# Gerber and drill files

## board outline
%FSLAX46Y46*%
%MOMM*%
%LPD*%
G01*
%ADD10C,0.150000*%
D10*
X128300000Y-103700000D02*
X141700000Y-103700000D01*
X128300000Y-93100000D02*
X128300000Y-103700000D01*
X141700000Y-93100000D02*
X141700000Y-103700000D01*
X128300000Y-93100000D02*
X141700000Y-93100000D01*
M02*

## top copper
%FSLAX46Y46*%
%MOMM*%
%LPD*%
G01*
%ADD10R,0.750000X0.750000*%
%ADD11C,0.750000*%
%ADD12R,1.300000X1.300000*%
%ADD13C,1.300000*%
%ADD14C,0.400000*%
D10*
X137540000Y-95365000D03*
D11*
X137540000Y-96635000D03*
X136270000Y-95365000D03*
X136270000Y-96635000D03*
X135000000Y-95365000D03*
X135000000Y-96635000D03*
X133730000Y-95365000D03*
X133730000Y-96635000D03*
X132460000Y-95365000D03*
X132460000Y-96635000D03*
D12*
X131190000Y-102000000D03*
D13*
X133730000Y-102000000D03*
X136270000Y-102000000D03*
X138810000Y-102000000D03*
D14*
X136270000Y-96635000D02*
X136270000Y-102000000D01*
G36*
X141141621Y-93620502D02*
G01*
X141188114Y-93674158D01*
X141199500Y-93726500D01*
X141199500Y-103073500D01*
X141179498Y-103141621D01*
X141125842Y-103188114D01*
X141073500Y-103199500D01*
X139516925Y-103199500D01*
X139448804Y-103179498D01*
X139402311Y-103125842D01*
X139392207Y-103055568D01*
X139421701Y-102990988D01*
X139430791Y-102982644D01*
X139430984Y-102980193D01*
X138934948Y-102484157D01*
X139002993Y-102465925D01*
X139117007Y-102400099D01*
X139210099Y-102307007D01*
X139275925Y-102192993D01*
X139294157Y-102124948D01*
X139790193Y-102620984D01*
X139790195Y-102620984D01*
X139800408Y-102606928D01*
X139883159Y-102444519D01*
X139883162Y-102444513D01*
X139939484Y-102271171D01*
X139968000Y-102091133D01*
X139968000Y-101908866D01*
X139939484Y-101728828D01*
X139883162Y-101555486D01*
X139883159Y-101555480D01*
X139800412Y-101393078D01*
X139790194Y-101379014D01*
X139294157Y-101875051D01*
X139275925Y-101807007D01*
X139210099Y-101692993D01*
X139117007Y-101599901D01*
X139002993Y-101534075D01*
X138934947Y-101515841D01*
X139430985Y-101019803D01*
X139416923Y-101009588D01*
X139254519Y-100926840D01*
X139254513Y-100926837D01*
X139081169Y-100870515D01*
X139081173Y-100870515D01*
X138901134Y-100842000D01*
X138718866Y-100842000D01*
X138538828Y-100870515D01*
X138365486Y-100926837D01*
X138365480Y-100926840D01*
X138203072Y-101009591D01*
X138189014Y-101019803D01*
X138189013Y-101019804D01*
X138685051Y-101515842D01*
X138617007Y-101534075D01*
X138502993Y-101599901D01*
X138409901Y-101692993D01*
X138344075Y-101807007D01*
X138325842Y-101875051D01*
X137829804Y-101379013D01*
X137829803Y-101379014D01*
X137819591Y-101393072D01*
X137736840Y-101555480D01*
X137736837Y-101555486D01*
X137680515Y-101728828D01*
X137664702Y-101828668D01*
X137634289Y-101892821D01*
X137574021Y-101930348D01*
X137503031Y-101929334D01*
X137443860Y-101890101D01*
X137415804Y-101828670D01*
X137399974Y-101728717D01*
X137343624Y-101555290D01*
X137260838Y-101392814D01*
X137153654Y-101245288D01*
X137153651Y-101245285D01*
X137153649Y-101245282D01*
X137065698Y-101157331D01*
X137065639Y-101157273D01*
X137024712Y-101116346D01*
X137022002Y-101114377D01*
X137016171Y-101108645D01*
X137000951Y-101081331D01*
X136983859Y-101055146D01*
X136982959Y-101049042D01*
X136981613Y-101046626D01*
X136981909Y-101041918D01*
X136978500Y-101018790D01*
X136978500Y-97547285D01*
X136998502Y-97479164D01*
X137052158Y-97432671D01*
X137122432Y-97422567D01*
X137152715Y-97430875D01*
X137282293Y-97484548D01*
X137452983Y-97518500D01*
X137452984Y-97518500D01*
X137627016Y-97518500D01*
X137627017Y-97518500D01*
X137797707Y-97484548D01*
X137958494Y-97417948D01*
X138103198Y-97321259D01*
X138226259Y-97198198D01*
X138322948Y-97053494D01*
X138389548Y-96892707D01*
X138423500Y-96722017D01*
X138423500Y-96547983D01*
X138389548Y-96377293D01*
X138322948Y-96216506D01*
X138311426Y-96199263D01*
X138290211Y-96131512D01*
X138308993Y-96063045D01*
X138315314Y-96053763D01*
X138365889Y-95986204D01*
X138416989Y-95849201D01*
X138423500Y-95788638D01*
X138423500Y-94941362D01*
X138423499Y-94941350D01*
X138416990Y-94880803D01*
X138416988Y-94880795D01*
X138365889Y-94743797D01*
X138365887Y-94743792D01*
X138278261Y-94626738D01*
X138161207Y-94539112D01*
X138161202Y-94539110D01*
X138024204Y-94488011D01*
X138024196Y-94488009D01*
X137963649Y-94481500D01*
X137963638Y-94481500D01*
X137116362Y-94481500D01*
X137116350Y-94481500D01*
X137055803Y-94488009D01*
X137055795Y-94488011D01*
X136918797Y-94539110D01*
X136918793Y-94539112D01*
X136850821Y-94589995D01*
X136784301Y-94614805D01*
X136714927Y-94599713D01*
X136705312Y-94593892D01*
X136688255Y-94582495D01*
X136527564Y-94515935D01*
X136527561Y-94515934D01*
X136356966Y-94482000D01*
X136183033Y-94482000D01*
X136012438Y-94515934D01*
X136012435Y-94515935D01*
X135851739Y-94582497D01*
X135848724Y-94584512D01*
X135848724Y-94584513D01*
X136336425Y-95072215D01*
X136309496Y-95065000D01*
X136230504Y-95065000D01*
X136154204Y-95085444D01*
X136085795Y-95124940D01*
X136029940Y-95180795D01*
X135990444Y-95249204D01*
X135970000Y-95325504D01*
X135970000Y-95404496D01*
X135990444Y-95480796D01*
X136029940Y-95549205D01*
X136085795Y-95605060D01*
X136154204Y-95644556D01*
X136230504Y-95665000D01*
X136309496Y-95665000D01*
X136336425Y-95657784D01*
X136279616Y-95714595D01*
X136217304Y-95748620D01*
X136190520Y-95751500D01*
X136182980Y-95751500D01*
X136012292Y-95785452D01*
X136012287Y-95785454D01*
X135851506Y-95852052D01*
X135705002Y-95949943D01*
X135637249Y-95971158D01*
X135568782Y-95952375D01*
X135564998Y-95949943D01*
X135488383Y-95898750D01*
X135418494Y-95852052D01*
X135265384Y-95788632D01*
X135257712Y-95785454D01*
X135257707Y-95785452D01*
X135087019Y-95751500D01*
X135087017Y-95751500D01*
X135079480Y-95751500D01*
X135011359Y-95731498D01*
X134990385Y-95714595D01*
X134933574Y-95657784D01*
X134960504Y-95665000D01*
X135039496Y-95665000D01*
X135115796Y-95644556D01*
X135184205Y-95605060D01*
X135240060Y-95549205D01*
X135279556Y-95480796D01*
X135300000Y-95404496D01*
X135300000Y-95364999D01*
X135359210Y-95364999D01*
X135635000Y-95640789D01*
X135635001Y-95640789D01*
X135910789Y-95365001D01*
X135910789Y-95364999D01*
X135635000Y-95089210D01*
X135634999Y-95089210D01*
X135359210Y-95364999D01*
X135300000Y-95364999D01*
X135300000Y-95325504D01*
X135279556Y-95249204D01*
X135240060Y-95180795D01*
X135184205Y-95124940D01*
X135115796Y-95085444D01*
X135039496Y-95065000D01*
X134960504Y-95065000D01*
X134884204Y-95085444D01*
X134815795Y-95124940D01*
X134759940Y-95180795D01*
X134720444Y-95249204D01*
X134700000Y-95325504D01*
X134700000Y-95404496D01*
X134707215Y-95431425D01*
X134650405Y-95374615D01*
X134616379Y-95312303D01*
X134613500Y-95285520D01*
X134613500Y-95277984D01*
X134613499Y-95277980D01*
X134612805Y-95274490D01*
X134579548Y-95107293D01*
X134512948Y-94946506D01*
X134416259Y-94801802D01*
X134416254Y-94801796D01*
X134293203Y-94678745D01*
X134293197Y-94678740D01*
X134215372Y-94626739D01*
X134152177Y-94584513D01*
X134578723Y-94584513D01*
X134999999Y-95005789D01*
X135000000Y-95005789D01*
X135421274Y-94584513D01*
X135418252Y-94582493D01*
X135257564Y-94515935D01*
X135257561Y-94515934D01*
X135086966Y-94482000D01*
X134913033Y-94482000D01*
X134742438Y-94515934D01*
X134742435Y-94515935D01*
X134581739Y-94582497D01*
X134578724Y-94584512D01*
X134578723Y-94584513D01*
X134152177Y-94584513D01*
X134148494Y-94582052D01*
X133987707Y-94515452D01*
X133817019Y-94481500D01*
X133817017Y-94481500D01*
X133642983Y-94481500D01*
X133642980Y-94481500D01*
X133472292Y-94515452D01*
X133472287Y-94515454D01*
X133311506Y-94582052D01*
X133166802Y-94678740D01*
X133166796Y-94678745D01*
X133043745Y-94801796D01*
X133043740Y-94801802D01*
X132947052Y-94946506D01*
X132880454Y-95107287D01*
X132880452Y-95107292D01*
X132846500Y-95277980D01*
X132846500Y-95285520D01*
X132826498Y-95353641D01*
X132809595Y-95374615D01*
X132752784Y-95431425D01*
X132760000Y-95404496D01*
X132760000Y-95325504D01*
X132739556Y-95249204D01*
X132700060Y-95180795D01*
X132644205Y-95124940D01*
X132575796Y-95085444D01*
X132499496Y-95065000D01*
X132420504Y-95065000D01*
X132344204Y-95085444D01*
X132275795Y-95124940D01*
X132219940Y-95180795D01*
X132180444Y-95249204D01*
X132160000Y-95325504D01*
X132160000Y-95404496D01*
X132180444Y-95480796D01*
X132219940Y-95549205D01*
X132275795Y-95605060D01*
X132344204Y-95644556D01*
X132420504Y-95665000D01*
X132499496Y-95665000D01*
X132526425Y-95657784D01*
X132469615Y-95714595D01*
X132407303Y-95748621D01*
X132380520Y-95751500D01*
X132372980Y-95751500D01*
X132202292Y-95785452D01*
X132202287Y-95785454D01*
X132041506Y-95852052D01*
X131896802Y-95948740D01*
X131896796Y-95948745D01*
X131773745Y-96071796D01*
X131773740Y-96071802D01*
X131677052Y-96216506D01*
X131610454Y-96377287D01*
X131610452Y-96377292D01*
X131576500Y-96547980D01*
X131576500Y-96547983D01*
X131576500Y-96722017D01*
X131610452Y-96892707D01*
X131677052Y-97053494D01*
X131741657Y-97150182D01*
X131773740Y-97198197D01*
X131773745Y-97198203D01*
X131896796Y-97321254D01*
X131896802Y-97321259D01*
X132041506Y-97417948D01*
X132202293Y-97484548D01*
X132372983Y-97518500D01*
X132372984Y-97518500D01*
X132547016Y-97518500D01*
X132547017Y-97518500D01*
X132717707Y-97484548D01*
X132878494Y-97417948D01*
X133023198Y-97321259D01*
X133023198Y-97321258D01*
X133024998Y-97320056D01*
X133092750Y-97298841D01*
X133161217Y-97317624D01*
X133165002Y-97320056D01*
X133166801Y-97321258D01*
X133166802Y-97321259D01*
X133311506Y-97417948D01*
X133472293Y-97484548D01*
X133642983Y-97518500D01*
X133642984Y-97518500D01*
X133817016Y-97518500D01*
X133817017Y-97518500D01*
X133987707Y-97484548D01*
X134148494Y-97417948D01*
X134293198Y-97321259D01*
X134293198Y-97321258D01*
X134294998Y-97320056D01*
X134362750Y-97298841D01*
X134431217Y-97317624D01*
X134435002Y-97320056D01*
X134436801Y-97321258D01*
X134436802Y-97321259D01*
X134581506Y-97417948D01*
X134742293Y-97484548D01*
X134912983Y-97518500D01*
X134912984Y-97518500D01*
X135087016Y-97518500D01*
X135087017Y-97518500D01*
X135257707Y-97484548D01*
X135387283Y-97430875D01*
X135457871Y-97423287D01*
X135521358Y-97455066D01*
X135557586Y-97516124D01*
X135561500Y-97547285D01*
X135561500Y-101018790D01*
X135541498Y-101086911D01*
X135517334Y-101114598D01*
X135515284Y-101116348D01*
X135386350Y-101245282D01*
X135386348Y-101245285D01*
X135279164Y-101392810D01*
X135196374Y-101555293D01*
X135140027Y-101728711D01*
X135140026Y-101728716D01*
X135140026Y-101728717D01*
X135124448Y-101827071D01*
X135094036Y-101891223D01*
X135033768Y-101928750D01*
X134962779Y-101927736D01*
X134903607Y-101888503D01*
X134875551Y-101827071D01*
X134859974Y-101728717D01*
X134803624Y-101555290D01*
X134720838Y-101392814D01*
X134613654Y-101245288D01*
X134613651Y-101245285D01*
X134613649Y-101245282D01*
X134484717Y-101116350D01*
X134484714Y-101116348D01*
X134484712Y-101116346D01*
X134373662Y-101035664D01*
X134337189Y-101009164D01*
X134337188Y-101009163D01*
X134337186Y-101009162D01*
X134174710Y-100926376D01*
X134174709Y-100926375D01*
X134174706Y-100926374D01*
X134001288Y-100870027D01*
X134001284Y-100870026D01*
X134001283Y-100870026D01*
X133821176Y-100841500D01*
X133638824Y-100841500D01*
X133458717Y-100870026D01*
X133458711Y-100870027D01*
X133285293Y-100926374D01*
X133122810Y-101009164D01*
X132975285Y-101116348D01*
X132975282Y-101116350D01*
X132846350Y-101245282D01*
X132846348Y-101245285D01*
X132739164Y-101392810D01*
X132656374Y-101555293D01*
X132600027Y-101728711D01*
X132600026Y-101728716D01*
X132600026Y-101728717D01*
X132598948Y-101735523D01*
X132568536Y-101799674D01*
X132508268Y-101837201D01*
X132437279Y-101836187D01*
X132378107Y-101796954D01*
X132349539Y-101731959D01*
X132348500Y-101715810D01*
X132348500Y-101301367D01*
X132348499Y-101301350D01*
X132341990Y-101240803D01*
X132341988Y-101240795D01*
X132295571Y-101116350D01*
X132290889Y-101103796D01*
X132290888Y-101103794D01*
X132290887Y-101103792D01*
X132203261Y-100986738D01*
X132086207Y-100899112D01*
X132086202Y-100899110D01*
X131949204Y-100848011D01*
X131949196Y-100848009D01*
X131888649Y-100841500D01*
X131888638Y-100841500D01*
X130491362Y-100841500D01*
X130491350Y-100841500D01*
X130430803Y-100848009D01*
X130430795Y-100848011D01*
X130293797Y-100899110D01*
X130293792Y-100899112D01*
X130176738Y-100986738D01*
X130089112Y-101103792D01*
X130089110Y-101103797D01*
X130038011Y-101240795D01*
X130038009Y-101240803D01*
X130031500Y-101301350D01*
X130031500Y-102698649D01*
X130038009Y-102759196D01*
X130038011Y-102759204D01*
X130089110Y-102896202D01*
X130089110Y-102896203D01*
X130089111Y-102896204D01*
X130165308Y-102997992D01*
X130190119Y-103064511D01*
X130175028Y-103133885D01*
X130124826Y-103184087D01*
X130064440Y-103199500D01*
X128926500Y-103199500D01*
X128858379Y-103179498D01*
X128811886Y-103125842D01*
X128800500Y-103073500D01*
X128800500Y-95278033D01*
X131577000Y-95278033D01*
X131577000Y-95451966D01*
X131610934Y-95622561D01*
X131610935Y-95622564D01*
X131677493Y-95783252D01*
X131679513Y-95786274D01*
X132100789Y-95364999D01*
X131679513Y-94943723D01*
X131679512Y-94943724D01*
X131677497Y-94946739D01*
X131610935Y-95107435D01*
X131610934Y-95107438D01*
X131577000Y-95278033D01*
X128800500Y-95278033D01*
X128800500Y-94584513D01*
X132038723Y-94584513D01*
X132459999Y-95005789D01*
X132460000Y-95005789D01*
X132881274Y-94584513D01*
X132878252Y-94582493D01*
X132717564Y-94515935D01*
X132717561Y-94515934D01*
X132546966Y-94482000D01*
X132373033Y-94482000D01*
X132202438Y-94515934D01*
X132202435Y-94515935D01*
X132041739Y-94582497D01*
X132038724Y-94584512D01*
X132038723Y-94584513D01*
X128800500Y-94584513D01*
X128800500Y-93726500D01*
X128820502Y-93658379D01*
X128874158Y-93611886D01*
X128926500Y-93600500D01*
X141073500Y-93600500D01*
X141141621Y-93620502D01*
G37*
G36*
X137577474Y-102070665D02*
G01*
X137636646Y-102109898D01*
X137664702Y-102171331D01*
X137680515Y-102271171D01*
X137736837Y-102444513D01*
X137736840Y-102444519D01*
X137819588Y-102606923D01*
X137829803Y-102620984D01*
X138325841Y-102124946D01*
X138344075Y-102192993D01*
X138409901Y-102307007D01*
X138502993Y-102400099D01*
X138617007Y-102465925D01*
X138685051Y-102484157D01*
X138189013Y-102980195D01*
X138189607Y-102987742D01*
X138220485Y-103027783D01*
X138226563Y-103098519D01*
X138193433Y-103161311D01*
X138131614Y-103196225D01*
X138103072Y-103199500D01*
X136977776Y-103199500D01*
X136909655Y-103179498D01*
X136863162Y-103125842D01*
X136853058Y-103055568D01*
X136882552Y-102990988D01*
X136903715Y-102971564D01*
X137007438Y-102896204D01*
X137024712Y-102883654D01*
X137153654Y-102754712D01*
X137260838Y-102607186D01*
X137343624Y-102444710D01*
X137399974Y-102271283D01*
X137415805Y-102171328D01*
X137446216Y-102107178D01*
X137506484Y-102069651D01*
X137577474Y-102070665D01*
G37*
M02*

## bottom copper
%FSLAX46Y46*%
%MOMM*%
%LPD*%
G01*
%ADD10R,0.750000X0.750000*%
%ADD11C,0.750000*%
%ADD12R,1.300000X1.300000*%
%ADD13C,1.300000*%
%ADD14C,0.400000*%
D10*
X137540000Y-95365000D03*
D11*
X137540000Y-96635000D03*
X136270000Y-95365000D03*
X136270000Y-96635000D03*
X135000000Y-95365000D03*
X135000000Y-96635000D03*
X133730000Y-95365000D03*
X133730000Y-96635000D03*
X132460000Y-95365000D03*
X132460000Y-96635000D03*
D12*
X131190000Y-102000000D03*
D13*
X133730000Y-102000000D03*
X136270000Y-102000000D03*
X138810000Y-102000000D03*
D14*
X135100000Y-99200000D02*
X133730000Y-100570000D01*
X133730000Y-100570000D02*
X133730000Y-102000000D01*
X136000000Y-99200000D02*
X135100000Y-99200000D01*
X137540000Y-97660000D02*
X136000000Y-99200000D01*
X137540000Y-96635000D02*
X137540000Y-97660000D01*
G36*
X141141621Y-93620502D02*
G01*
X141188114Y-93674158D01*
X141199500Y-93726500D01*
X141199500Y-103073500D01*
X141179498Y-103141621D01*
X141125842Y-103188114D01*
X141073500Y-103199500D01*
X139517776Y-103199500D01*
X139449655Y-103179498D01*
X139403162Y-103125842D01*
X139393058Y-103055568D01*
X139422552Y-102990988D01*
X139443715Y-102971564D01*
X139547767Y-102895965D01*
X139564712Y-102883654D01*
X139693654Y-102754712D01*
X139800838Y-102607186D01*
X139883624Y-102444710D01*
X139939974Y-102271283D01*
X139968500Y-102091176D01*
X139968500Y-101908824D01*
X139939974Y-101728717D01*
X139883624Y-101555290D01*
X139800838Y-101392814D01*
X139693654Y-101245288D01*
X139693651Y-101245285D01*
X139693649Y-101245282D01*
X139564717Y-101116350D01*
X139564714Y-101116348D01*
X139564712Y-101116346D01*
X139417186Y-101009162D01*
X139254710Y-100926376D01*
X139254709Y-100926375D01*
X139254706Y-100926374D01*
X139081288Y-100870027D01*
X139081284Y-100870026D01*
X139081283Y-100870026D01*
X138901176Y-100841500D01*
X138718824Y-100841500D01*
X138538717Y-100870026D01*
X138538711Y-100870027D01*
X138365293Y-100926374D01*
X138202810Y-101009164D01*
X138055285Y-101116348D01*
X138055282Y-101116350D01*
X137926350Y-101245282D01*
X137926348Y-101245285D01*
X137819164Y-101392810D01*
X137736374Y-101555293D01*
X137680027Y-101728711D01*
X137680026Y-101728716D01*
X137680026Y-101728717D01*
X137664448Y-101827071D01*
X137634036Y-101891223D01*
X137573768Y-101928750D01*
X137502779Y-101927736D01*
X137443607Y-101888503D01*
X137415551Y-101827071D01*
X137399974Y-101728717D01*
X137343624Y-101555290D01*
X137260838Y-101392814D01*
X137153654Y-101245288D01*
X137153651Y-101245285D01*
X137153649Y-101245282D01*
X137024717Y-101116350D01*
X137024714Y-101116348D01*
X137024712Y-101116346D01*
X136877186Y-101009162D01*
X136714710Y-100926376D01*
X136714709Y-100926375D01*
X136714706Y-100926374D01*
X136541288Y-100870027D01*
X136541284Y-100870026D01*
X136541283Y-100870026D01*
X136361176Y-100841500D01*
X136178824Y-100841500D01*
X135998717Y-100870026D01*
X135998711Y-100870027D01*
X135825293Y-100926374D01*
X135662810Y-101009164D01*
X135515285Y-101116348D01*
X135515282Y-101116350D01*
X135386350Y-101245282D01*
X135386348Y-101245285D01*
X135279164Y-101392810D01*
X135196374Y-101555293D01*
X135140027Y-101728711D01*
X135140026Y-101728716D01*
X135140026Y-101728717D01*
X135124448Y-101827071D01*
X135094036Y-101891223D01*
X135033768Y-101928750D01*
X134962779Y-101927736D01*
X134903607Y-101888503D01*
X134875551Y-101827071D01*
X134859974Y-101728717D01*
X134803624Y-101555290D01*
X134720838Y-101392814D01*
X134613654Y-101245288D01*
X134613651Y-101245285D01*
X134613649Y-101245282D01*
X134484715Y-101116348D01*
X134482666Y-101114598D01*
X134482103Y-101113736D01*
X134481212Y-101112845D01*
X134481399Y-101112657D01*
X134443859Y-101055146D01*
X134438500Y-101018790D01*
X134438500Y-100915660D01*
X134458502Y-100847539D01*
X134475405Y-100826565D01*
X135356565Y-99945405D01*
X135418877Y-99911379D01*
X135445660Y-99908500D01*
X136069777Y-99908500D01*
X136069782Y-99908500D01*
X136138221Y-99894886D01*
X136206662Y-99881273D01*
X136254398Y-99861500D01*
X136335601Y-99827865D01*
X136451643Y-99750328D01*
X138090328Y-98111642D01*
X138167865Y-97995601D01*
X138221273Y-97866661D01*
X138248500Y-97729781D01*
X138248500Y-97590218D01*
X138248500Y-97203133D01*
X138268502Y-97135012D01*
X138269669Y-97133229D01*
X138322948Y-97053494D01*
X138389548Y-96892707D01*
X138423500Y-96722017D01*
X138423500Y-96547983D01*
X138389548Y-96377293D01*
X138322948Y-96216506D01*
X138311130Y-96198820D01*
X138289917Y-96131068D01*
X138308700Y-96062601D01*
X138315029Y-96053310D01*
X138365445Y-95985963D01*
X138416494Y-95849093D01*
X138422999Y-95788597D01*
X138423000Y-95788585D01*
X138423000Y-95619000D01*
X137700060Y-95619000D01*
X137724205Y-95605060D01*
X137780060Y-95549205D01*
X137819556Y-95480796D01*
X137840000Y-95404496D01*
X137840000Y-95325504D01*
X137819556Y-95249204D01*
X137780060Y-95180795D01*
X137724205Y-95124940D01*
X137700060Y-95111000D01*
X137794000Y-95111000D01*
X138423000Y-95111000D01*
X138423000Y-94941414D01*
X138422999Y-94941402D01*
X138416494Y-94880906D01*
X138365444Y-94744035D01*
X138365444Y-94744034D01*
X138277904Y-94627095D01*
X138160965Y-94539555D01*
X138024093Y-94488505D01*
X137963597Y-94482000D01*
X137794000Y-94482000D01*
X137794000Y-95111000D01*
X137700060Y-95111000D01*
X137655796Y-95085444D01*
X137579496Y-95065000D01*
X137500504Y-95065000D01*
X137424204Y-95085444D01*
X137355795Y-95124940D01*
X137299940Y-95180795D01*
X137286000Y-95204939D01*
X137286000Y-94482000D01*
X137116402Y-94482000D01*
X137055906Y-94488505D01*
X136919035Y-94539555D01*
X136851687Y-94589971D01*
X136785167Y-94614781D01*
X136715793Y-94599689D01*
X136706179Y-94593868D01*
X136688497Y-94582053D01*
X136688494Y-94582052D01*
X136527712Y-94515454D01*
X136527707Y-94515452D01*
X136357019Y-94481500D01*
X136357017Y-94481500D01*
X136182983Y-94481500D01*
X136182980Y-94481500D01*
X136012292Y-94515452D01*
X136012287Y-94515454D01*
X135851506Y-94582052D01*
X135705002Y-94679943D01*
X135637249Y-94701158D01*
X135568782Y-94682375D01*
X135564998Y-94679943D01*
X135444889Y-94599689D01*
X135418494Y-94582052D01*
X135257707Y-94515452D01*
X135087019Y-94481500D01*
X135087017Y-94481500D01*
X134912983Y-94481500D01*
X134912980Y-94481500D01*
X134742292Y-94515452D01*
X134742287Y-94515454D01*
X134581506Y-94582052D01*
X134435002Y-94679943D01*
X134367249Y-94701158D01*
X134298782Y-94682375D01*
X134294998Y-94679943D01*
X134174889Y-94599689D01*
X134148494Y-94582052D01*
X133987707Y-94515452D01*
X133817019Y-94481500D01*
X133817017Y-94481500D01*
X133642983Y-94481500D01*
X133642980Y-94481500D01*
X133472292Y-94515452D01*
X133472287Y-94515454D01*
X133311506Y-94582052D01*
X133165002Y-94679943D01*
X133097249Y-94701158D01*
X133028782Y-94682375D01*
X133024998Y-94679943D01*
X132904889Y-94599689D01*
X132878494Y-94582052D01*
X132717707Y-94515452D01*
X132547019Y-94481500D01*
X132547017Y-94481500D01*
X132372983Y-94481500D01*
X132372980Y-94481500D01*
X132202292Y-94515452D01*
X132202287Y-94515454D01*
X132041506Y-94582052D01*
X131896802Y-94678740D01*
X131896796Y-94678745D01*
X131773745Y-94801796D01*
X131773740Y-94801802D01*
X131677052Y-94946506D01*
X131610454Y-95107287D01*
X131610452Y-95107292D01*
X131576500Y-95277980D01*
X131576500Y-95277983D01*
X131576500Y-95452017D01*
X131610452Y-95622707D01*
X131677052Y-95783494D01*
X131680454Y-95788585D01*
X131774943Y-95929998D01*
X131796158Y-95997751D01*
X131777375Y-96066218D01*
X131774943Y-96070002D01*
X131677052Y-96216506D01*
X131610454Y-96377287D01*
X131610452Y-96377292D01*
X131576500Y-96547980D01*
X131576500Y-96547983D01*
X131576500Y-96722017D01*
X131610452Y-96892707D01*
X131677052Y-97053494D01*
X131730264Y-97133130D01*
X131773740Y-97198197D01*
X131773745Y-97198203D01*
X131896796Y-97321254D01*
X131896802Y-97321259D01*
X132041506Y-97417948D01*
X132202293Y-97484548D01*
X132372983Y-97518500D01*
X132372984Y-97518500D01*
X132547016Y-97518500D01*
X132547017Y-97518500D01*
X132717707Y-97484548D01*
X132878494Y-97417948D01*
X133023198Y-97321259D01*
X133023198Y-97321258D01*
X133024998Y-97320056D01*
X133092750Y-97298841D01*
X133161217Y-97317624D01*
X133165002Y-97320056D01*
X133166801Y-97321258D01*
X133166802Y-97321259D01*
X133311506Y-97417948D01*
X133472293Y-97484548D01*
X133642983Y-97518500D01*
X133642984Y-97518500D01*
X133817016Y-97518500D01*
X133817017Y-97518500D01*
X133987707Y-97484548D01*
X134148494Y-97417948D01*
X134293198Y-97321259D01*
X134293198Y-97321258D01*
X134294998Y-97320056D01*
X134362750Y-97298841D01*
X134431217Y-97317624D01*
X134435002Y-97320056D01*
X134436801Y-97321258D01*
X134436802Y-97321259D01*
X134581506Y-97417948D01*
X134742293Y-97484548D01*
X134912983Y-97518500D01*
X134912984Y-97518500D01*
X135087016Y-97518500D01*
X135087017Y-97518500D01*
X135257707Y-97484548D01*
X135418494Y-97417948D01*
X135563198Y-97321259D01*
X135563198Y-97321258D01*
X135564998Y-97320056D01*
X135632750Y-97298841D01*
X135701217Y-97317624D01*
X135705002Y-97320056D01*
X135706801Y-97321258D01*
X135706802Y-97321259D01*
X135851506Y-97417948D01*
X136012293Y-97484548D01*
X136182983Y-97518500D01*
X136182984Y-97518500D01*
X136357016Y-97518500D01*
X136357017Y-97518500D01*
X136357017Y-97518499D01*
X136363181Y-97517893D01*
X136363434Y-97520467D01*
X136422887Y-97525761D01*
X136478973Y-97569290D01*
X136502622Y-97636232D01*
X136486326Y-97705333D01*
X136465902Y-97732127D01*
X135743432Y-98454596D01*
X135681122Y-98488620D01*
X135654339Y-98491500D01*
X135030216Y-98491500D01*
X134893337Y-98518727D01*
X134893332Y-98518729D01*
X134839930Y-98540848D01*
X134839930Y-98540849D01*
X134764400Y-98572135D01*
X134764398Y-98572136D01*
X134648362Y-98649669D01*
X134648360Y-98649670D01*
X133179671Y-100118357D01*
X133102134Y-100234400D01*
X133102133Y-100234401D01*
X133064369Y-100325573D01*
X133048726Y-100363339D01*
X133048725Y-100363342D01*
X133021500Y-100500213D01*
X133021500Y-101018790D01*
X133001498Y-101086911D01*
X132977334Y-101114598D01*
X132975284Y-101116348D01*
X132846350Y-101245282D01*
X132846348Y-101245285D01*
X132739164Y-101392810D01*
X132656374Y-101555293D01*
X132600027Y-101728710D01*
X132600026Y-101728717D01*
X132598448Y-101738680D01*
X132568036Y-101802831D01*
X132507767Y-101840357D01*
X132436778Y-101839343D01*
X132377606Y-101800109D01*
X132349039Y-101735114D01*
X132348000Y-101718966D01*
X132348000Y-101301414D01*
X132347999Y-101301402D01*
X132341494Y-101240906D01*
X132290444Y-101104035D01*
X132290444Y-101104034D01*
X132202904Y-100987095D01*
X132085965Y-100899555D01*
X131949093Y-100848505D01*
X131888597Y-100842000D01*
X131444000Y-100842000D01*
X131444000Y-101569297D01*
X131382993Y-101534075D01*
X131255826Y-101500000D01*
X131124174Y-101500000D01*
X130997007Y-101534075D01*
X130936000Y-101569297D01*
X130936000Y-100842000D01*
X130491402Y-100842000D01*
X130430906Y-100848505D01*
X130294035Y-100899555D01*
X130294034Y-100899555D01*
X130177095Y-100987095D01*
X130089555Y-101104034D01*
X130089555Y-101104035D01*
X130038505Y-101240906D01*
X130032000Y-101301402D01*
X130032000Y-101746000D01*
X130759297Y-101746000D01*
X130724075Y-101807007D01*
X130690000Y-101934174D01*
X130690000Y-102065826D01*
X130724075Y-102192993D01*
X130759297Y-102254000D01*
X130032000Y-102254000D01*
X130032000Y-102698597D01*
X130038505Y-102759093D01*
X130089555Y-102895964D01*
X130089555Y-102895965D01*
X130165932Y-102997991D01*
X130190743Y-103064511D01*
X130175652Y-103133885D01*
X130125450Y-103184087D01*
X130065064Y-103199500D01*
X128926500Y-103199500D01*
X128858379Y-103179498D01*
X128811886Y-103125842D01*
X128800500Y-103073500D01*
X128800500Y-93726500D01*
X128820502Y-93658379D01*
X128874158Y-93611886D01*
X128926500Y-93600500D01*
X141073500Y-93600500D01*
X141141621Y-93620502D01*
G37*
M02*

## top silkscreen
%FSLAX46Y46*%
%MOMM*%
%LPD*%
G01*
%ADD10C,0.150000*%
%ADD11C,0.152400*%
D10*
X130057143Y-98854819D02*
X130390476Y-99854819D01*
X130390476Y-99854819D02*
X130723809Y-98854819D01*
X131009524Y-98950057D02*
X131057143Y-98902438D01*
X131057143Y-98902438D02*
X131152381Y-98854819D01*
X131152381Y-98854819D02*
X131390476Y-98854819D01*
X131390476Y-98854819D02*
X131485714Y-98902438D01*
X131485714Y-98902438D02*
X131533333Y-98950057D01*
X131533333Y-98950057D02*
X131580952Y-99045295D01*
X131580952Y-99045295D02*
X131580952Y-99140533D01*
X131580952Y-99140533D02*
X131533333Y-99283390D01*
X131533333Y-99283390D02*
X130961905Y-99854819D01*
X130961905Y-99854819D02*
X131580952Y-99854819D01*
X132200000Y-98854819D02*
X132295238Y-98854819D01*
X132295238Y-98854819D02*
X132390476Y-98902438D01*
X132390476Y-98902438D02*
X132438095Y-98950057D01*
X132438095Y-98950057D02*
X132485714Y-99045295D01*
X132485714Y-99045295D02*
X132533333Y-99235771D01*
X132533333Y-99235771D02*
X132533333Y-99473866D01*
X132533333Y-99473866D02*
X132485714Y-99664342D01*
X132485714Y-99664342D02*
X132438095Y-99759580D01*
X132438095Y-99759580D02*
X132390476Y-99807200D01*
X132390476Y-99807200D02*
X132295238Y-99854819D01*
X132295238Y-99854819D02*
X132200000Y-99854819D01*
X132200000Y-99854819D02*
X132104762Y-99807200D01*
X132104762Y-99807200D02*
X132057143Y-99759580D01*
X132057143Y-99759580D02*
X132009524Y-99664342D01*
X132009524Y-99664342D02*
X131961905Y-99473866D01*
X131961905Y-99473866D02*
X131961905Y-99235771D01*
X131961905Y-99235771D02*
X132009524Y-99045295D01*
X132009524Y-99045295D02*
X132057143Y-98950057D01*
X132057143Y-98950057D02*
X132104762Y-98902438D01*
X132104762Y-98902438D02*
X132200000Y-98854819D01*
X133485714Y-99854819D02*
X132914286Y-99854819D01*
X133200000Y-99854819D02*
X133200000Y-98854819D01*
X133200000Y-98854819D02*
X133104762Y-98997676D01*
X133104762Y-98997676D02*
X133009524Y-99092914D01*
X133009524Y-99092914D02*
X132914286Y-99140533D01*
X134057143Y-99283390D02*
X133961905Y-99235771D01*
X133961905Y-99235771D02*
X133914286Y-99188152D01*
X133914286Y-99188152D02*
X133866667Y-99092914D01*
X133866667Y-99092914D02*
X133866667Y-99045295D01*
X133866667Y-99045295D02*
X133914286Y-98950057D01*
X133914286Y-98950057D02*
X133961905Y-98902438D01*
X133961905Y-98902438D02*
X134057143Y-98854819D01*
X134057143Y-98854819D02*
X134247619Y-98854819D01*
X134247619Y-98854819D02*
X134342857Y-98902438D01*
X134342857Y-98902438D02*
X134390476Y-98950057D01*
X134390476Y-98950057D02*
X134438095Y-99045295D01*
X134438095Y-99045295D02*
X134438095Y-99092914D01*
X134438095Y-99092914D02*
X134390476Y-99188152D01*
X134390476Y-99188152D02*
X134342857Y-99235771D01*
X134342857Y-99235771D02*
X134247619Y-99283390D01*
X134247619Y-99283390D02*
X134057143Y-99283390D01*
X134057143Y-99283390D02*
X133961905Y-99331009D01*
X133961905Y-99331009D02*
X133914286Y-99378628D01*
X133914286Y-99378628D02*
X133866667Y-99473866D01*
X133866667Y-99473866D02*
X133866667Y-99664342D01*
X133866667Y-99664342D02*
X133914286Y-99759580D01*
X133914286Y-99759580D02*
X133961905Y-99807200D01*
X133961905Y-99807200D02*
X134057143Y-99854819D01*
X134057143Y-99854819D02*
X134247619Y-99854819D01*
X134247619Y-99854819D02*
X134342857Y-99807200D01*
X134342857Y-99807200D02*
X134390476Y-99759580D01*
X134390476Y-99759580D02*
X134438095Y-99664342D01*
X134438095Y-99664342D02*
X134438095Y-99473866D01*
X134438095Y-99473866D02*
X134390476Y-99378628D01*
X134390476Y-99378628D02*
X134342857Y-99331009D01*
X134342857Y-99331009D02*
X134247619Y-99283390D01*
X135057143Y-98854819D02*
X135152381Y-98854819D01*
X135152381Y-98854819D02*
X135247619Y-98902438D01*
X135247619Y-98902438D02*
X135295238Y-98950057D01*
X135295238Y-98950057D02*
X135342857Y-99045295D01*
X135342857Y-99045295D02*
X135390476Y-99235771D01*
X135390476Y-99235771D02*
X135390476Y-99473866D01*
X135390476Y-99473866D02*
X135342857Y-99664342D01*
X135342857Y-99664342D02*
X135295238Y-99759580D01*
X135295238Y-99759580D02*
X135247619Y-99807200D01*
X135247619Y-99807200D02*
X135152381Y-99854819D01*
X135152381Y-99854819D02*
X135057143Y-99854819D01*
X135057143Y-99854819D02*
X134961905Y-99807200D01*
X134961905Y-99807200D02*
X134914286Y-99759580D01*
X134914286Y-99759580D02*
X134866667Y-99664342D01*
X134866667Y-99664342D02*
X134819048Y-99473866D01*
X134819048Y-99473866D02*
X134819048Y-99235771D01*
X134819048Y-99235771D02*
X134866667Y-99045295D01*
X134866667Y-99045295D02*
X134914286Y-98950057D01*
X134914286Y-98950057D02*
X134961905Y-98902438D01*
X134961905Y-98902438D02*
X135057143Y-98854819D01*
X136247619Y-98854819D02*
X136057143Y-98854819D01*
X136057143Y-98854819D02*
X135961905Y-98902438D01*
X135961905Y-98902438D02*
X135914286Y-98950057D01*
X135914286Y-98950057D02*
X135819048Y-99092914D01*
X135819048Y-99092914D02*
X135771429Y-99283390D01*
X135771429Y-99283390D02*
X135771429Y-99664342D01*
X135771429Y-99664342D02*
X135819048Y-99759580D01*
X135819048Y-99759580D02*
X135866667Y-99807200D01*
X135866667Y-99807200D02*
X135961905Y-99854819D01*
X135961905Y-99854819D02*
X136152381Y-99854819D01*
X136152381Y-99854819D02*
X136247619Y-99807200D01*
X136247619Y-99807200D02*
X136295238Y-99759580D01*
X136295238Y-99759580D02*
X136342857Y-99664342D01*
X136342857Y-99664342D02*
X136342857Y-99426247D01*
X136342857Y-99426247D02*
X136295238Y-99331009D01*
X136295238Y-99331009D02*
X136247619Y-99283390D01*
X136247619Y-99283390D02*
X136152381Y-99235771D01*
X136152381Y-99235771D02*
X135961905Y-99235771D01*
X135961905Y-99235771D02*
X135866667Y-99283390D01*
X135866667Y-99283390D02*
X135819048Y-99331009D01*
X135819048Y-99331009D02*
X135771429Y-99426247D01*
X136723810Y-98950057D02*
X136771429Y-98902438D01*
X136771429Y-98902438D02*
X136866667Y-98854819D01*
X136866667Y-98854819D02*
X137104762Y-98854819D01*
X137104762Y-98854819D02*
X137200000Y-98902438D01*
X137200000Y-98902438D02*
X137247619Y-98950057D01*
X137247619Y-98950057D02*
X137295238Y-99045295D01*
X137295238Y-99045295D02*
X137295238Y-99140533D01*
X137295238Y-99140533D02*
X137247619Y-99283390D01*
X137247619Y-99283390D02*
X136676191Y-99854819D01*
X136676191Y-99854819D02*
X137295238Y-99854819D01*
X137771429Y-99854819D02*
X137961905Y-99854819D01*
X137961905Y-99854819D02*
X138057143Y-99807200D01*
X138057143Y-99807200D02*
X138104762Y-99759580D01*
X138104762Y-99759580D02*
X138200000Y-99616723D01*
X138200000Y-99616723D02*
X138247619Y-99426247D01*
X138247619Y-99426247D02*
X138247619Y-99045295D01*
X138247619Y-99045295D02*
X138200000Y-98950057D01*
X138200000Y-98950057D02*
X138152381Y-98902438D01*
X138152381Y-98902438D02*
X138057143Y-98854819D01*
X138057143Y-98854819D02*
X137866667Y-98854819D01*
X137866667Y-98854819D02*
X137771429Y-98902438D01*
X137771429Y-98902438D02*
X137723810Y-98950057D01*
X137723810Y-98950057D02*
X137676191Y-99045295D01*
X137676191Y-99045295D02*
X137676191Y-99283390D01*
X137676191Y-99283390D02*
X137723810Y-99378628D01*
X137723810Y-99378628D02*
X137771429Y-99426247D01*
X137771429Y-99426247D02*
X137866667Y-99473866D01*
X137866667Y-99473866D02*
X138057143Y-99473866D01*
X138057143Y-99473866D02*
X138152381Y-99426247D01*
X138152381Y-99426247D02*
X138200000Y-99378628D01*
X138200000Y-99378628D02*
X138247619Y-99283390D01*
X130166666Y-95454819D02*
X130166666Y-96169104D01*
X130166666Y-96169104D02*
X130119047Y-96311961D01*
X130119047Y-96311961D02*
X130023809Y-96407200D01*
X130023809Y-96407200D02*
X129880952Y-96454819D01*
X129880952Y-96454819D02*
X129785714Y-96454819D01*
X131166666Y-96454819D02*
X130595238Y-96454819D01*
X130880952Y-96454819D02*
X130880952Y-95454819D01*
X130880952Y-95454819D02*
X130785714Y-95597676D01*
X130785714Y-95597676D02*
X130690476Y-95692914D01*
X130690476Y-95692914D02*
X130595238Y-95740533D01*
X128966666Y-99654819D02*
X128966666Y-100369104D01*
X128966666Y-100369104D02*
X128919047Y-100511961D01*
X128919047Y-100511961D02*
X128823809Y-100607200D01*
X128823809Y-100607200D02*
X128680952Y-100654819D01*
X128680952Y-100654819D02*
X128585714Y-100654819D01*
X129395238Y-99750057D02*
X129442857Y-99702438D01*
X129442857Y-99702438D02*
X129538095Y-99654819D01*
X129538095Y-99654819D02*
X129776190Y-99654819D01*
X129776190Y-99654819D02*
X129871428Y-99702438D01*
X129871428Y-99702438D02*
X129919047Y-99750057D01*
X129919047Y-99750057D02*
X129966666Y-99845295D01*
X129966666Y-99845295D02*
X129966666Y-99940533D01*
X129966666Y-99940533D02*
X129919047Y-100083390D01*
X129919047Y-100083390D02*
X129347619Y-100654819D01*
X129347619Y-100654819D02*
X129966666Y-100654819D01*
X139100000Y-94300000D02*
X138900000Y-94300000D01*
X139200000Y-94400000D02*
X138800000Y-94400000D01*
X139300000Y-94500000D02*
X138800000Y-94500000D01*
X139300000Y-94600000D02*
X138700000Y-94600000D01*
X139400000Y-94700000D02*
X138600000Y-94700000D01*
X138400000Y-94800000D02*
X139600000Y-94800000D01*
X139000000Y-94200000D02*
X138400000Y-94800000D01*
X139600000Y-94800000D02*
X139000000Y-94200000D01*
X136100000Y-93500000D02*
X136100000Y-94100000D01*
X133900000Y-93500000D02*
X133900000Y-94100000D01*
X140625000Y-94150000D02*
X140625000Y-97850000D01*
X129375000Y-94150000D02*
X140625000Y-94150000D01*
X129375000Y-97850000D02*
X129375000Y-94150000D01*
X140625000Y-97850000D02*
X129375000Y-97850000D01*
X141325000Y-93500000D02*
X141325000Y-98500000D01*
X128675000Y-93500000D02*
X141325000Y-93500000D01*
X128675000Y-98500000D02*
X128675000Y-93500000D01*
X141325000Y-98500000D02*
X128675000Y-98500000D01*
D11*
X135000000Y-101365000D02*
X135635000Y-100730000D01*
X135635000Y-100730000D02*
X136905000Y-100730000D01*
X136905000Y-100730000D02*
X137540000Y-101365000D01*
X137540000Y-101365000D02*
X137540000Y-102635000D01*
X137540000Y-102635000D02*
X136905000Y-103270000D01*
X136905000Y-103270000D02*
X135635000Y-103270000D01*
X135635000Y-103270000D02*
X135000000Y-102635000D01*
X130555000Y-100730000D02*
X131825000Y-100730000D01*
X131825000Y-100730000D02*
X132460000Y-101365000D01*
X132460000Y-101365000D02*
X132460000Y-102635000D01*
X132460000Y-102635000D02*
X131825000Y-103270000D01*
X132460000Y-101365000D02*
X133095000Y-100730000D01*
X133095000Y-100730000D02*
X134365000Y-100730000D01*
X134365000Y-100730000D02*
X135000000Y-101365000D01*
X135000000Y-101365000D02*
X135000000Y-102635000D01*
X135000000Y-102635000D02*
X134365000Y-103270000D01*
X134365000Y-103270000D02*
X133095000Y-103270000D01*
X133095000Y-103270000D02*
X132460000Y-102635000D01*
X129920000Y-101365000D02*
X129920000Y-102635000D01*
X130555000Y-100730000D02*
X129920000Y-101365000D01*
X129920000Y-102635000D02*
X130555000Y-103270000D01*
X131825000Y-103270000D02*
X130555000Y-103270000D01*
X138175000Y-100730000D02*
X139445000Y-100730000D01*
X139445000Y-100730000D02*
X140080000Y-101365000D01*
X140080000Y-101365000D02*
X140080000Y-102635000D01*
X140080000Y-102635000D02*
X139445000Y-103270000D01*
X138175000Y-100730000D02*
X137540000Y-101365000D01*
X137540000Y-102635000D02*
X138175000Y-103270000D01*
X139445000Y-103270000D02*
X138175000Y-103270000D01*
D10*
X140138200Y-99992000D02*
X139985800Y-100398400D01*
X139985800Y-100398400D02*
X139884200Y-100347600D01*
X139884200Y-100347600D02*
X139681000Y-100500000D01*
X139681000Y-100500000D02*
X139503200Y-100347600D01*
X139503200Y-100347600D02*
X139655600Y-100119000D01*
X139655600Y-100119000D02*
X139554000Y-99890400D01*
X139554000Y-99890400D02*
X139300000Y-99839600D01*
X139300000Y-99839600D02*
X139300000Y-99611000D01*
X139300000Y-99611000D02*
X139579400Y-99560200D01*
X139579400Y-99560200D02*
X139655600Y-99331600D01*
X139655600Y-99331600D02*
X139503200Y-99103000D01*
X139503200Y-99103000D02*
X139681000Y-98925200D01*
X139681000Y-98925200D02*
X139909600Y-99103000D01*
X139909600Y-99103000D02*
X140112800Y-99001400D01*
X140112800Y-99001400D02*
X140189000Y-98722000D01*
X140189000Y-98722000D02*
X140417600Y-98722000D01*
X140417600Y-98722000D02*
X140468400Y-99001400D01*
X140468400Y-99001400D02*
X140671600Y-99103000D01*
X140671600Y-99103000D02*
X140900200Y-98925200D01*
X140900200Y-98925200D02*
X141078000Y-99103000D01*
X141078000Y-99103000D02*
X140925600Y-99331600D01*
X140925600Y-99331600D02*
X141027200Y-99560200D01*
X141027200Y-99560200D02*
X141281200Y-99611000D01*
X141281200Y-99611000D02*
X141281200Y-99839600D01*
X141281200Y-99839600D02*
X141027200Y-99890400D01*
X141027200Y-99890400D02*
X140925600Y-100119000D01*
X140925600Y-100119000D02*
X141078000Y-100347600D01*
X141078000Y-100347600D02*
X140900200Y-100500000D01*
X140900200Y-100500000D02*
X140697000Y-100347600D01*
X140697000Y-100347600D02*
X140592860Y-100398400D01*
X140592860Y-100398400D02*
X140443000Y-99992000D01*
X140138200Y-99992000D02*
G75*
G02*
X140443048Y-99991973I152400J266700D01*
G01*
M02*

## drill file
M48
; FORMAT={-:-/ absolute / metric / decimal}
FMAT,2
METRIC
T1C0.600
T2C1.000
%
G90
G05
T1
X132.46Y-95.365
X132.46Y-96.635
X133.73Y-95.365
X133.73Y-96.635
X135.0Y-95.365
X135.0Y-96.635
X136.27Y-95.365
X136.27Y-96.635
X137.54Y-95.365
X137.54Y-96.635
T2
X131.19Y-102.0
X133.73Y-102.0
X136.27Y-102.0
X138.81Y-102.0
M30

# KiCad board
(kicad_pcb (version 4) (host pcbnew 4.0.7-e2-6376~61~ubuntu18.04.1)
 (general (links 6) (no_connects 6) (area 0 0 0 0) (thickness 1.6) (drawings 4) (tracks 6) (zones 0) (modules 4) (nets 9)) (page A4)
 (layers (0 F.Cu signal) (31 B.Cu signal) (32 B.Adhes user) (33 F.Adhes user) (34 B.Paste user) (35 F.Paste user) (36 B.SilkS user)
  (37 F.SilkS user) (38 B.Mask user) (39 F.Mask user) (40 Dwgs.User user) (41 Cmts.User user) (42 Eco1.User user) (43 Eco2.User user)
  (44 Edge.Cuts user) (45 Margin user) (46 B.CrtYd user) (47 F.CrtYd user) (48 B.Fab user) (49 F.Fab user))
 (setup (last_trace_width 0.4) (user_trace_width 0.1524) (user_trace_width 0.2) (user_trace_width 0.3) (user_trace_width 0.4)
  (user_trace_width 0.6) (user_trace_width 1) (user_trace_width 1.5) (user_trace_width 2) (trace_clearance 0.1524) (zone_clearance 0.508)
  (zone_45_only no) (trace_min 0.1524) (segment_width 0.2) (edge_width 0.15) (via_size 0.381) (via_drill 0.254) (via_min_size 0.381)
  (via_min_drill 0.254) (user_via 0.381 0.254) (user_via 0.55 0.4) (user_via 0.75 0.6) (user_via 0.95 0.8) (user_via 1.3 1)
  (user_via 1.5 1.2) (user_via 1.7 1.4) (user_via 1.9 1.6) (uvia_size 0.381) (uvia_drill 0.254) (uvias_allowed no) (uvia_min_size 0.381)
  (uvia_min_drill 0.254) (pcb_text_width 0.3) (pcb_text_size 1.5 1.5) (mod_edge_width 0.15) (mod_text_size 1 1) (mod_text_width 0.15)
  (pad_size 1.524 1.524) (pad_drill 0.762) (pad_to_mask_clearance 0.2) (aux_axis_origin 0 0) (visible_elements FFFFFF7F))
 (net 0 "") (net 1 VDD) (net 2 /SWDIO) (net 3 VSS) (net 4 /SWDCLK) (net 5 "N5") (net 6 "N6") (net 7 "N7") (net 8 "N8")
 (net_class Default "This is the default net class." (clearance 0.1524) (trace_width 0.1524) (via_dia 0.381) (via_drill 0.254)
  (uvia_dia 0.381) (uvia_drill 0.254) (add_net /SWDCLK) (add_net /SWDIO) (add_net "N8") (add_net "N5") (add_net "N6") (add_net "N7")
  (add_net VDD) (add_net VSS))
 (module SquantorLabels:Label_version (layer F.Cu) (at 135 99.4)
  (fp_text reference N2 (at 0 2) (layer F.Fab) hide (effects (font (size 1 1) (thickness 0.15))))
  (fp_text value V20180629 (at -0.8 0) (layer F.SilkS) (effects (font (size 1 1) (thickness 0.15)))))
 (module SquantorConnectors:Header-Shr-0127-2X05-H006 (layer F.Cu) (at 135 96 180)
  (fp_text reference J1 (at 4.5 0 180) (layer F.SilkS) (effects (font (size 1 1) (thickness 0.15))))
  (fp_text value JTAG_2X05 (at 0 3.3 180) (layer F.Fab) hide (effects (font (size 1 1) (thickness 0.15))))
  (fp_line (start -4.1 1.7) (end -3.9 1.7) (layer F.SilkS) (width 0.15))
  (fp_line (start -4.2 1.6) (end -3.8 1.6) (layer F.SilkS) (width 0.15))
  (fp_line (start -4.3 1.5) (end -3.8 1.5) (layer F.SilkS) (width 0.15))
  (fp_line (start -4.3 1.4) (end -3.7 1.4) (layer F.SilkS) (width 0.15))
  (fp_line (start -4.4 1.3) (end -3.6 1.3) (layer F.SilkS) (width 0.15))
  (fp_line (start -3.4 1.2) (end -4.6 1.2) (layer F.SilkS) (width 0.15))
  (fp_line (start -4 1.8) (end -3.4 1.2) (layer F.SilkS) (width 0.15))
  (fp_line (start -4.6 1.2) (end -4 1.8) (layer F.SilkS) (width 0.15))
  (fp_line (start -1.1 2.5) (end -1.1 1.9) (layer F.SilkS) (width 0.15))
  (fp_line (start 1.1 2.5) (end 1.1 1.9) (layer F.SilkS) (width 0.15))
  (fp_line (start -5.625 1.85) (end -5.625 -1.85) (layer F.SilkS) (width 0.15))
  (fp_line (start 5.625 1.85) (end -5.625 1.85) (layer F.SilkS) (width 0.15))
  (fp_line (start 5.625 -1.85) (end 5.625 1.85) (layer F.SilkS) (width 0.15))
  (fp_line (start -5.625 -1.85) (end 5.625 -1.85) (layer F.SilkS) (width 0.15))
  (fp_line (start -6.325 2.5) (end -6.325 -2.5) (layer F.SilkS) (width 0.15))
  (fp_line (start 6.325 2.5) (end -6.325 2.5) (layer F.SilkS) (width 0.15))
  (fp_line (start 6.325 -2.5) (end 6.325 2.5) (layer F.SilkS) (width 0.15))
  (fp_line (start -6.325 -2.5) (end 6.325 -2.5) (layer F.SilkS) (width 0.15))
  (pad 1 thru_hole rect (at -2.54 0.635 180) (size 0.75 0.75) (drill 0.6) (layers *.Cu *.Mask) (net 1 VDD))
  (pad 2 thru_hole circle (at -2.54 -0.635 180) (size 0.75 0.75) (drill 0.6) (layers *.Cu *.Mask) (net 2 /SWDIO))
  (pad 3 thru_hole circle (at -1.27 0.635 180) (size 0.75 0.75) (drill 0.6) (layers *.Cu *.Mask) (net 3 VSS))
  (pad 4 thru_hole circle (at -1.27 -0.635 180) (size 0.75 0.75) (drill 0.6) (layers *.Cu *.Mask) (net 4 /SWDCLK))
  (pad 5 thru_hole circle (at 0 0.635 180) (size 0.75 0.75) (drill 0.6) (layers *.Cu *.Mask) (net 3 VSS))
  (pad 6 thru_hole circle (at 0 -0.635 180) (size 0.75 0.75) (drill 0.6) (layers *.Cu *.Mask) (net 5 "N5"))
  (pad 7 thru_hole circle (at 1.27 0.635 180) (size 0.75 0.75) (drill 0.6) (layers *.Cu *.Mask) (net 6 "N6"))
  (pad 8 thru_hole circle (at 1.27 -0.635 180) (size 0.75 0.75) (drill 0.6) (layers *.Cu *.Mask) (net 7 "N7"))
  (pad 9 thru_hole circle (at 2.54 0.635 180) (size 0.75 0.75) (drill 0.6) (layers *.Cu *.Mask) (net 3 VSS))
  (pad 10 thru_hole circle (at 2.54 -0.635 180) (size 0.75 0.75) (drill 0.6) (layers *.Cu *.Mask) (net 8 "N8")))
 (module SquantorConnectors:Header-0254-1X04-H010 (layer F.Cu) (at 135 102)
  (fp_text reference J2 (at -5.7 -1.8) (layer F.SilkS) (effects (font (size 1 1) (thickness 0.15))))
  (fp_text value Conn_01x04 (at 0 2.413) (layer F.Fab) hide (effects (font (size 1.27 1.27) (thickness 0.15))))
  (fp_line (start 0 -0.635) (end 0.635 -1.27) (layer F.SilkS) (width 0.1524))
  (fp_line (start 0.635 -1.27) (end 1.905 -1.27) (layer F.SilkS) (width 0.1524))
  (fp_line (start 1.905 -1.27) (end 2.54 -0.635) (layer F.SilkS) (width 0.1524))
  (fp_line (start 2.54 -0.635) (end 2.54 0.635) (layer F.SilkS) (width 0.1524))
  (fp_line (start 2.54 0.635) (end 1.905 1.27) (layer F.SilkS) (width 0.1524))
  (fp_line (start 1.905 1.27) (end 0.635 1.27) (layer F.SilkS) (width 0.1524))
  (fp_line (start 0.635 1.27) (end 0 0.635) (layer F.SilkS) (width 0.1524))
  (fp_line (start -4.445 -1.27) (end -3.175 -1.27) (layer F.SilkS) (width 0.1524))
  (fp_line (start -3.175 -1.27) (end -2.54 -0.635) (layer F.SilkS) (width 0.1524))
  (fp_line (start -2.54 -0.635) (end -2.54 0.635) (layer F.SilkS) (width 0.1524))
  (fp_line (start -2.54 0.635) (end -3.175 1.27) (layer F.SilkS) (width 0.1524))
  (fp_line (start -2.54 -0.635) (end -1.905 -1.27) (layer F.SilkS) (width 0.1524))
  (fp_line (start -1.905 -1.27) (end -0.635 -1.27) (layer F.SilkS) (width 0.1524))
  (fp_line (start -0.635 -1.27) (end 0 -0.635) (layer F.SilkS) (width 0.1524))
  (fp_line (start 0 -0.635) (end 0 0.635) (layer F.SilkS) (width 0.1524))
  (fp_line (start 0 0.635) (end -0.635 1.27) (layer F.SilkS) (width 0.1524))
  (fp_line (start -0.635 1.27) (end -1.905 1.27) (layer F.SilkS) (width 0.1524))
  (fp_line (start -1.905 1.27) (end -2.54 0.635) (layer F.SilkS) (width 0.1524))
  (fp_line (start -5.08 -0.635) (end -5.08 0.635) (layer F.SilkS) (width 0.1524))
  (fp_line (start -4.445 -1.27) (end -5.08 -0.635) (layer F.SilkS) (width 0.1524))
  (fp_line (start -5.08 0.635) (end -4.445 1.27) (layer F.SilkS) (width 0.1524))
  (fp_line (start -3.175 1.27) (end -4.445 1.27) (layer F.SilkS) (width 0.1524))
  (fp_line (start 3.175 -1.27) (end 4.445 -1.27) (layer F.SilkS) (width 0.1524))
  (fp_line (start 4.445 -1.27) (end 5.08 -0.635) (layer F.SilkS) (width 0.1524))
  (fp_line (start 5.08 -0.635) (end 5.08 0.635) (layer F.SilkS) (width 0.1524))
  (fp_line (start 5.08 0.635) (end 4.445 1.27) (layer F.SilkS) (width 0.1524))
  (fp_line (start 3.175 -1.27) (end 2.54 -0.635) (layer F.SilkS) (width 0.1524))
  (fp_line (start 2.54 0.635) (end 3.175 1.27) (layer F.SilkS) (width 0.1524))
  (fp_line (start 4.445 1.27) (end 3.175 1.27) (layer F.SilkS) (width 0.1524))
  (pad 1 thru_hole rect (at -3.81 0 180) (size 1.3 1.3) (drill 1) (layers *.Cu *.Mask) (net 1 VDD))
  (pad 2 thru_hole circle (at -1.27 0 180) (size 1.3 1.3) (drill 1) (layers *.Cu *.Mask) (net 2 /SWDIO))
  (pad 3 thru_hole circle (at 1.27 0 180) (size 1.3 1.3) (drill 1) (layers *.Cu *.Mask) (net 4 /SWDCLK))
  (pad 4 thru_hole circle (at 3.81 0 180) (size 1.3 1.3) (drill 1) (layers *.Cu *.Mask) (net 3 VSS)))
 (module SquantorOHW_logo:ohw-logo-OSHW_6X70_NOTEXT (layer F.Cu) (at 140.3 99.7)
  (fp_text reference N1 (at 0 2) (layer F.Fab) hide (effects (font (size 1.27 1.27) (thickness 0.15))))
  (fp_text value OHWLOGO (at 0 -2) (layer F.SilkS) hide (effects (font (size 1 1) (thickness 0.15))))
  (fp_line (start -0.1618 0.292) (end -0.3142 0.6984) (layer F.SilkS) (width 0.15))
  (fp_line (start -0.3142 0.6984) (end -0.4158 0.6476) (layer F.SilkS) (width 0.15))
  (fp_line (start -0.4158 0.6476) (end -0.619 0.8) (layer F.SilkS) (width 0.15))
  (fp_line (start -0.619 0.8) (end -0.7968 0.6476) (layer F.SilkS) (width 0.15))
  (fp_line (start -0.7968 0.6476) (end -0.6444 0.419) (layer F.SilkS) (width 0.15))
  (fp_line (start -0.6444 0.419) (end -0.746 0.1904) (layer F.SilkS) (width 0.15))
  (fp_line (start -0.746 0.1904) (end -1 0.1396) (layer F.SilkS) (width 0.15))
  (fp_line (start -1 0.1396) (end -1 -0.089) (layer F.SilkS) (width 0.15))
  (fp_line (start -1 -0.089) (end -0.7206 -0.1398) (layer F.SilkS) (width 0.15))
  (fp_line (start -0.7206 -0.1398) (end -0.6444 -0.3684) (layer F.SilkS) (width 0.15))
  (fp_line (start -0.6444 -0.3684) (end -0.7968 -0.597) (layer F.SilkS) (width 0.15))
  (fp_line (start -0.7968 -0.597) (end -0.619 -0.7748) (layer F.SilkS) (width 0.15))
  (fp_line (start -0.619 -0.7748) (end -0.3904 -0.597) (layer F.SilkS) (width 0.15))
  (fp_line (start -0.3904 -0.597) (end -0.1872 -0.6986) (layer F.SilkS) (width 0.15))
  (fp_line (start -0.1872 -0.6986) (end -0.111 -0.978) (layer F.SilkS) (width 0.15))
  (fp_line (start -0.111 -0.978) (end 0.1176 -0.978) (layer F.SilkS) (width 0.15))
  (fp_line (start 0.1176 -0.978) (end 0.1684 -0.6986) (layer F.SilkS) (width 0.15))
  (fp_line (start 0.1684 -0.6986) (end 0.3716 -0.597) (layer F.SilkS) (width 0.15))
  (fp_line (start 0.3716 -0.597) (end 0.6002 -0.7748) (layer F.SilkS) (width 0.15))
  (fp_line (start 0.6002 -0.7748) (end 0.778 -0.597) (layer F.SilkS) (width 0.15))
  (fp_line (start 0.778 -0.597) (end 0.6256 -0.3684) (layer F.SilkS) (width 0.15))
  (fp_line (start 0.6256 -0.3684) (end 0.7272 -0.1398) (layer F.SilkS) (width 0.15))
  (fp_line (start 0.7272 -0.1398) (end 0.9812 -0.089) (layer F.SilkS) (width 0.15))
  (fp_line (start 0.9812 -0.089) (end 0.9812 0.1396) (layer F.SilkS) (width 0.15))
  (fp_line (start 0.9812 0.1396) (end 0.7272 0.1904) (layer F.SilkS) (width 0.15))
  (fp_line (start 0.7272 0.1904) (end 0.6256 0.419) (layer F.SilkS) (width 0.15))
  (fp_line (start 0.6256 0.419) (end 0.778 0.6476) (layer F.SilkS) (width 0.15))
  (fp_line (start 0.778 0.6476) (end 0.6002 0.8) (layer F.SilkS) (width 0.15))
  (fp_line (start 0.6002 0.8) (end 0.397 0.6476) (layer F.SilkS) (width 0.15))
  (fp_line (start 0.397 0.6476) (end 0.29286 0.6984) (layer F.SilkS) (width 0.15))
  (fp_line (start 0.29286 0.6984) (end 0.143 0.292) (layer F.SilkS) (width 0.15))
  (fp_arc (start -0.0094 0.0253) (end -0.1618 0.292) (angle 300.5) (layer F.SilkS) (width 0.15)))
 (gr_line (start 128.3 103.7) (end 141.7 103.7) (layer Edge.Cuts) (width 0.15))
 (gr_line (start 128.3 93.1) (end 128.3 103.7) (layer Edge.Cuts) (width 0.15))
 (gr_line (start 141.7 93.1) (end 141.7 103.7) (layer Edge.Cuts) (width 0.15))
 (gr_line (start 128.3 93.1) (end 141.7 93.1) (layer Edge.Cuts) (width 0.15))
 (segment (start 135.1 99.2) (end 133.73 100.57) (width 0.4) (layer B.Cu) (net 2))
 (segment (start 133.73 100.57) (end 133.73 102) (width 0.4) (layer B.Cu) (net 2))
 (segment (start 136 99.2) (end 135.1 99.2) (width 0.4) (layer B.Cu) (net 2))
 (segment (start 137.54 97.66) (end 136 99.2) (width 0.4) (layer B.Cu) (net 2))
 (segment (start 137.54 96.635) (end 137.54 97.66) (width 0.4) (layer B.Cu) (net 2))
 (segment (start 136.27 96.635) (end 136.27 102) (width 0.4) (layer F.Cu) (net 4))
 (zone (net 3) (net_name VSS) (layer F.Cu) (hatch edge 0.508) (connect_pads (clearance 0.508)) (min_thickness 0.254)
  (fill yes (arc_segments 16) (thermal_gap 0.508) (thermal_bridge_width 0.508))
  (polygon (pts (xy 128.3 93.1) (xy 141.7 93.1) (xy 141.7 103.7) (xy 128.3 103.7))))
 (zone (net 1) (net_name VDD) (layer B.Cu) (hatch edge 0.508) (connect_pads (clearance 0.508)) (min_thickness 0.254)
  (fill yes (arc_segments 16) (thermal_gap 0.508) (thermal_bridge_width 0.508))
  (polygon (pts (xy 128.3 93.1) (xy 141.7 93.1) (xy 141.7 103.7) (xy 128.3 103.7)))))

